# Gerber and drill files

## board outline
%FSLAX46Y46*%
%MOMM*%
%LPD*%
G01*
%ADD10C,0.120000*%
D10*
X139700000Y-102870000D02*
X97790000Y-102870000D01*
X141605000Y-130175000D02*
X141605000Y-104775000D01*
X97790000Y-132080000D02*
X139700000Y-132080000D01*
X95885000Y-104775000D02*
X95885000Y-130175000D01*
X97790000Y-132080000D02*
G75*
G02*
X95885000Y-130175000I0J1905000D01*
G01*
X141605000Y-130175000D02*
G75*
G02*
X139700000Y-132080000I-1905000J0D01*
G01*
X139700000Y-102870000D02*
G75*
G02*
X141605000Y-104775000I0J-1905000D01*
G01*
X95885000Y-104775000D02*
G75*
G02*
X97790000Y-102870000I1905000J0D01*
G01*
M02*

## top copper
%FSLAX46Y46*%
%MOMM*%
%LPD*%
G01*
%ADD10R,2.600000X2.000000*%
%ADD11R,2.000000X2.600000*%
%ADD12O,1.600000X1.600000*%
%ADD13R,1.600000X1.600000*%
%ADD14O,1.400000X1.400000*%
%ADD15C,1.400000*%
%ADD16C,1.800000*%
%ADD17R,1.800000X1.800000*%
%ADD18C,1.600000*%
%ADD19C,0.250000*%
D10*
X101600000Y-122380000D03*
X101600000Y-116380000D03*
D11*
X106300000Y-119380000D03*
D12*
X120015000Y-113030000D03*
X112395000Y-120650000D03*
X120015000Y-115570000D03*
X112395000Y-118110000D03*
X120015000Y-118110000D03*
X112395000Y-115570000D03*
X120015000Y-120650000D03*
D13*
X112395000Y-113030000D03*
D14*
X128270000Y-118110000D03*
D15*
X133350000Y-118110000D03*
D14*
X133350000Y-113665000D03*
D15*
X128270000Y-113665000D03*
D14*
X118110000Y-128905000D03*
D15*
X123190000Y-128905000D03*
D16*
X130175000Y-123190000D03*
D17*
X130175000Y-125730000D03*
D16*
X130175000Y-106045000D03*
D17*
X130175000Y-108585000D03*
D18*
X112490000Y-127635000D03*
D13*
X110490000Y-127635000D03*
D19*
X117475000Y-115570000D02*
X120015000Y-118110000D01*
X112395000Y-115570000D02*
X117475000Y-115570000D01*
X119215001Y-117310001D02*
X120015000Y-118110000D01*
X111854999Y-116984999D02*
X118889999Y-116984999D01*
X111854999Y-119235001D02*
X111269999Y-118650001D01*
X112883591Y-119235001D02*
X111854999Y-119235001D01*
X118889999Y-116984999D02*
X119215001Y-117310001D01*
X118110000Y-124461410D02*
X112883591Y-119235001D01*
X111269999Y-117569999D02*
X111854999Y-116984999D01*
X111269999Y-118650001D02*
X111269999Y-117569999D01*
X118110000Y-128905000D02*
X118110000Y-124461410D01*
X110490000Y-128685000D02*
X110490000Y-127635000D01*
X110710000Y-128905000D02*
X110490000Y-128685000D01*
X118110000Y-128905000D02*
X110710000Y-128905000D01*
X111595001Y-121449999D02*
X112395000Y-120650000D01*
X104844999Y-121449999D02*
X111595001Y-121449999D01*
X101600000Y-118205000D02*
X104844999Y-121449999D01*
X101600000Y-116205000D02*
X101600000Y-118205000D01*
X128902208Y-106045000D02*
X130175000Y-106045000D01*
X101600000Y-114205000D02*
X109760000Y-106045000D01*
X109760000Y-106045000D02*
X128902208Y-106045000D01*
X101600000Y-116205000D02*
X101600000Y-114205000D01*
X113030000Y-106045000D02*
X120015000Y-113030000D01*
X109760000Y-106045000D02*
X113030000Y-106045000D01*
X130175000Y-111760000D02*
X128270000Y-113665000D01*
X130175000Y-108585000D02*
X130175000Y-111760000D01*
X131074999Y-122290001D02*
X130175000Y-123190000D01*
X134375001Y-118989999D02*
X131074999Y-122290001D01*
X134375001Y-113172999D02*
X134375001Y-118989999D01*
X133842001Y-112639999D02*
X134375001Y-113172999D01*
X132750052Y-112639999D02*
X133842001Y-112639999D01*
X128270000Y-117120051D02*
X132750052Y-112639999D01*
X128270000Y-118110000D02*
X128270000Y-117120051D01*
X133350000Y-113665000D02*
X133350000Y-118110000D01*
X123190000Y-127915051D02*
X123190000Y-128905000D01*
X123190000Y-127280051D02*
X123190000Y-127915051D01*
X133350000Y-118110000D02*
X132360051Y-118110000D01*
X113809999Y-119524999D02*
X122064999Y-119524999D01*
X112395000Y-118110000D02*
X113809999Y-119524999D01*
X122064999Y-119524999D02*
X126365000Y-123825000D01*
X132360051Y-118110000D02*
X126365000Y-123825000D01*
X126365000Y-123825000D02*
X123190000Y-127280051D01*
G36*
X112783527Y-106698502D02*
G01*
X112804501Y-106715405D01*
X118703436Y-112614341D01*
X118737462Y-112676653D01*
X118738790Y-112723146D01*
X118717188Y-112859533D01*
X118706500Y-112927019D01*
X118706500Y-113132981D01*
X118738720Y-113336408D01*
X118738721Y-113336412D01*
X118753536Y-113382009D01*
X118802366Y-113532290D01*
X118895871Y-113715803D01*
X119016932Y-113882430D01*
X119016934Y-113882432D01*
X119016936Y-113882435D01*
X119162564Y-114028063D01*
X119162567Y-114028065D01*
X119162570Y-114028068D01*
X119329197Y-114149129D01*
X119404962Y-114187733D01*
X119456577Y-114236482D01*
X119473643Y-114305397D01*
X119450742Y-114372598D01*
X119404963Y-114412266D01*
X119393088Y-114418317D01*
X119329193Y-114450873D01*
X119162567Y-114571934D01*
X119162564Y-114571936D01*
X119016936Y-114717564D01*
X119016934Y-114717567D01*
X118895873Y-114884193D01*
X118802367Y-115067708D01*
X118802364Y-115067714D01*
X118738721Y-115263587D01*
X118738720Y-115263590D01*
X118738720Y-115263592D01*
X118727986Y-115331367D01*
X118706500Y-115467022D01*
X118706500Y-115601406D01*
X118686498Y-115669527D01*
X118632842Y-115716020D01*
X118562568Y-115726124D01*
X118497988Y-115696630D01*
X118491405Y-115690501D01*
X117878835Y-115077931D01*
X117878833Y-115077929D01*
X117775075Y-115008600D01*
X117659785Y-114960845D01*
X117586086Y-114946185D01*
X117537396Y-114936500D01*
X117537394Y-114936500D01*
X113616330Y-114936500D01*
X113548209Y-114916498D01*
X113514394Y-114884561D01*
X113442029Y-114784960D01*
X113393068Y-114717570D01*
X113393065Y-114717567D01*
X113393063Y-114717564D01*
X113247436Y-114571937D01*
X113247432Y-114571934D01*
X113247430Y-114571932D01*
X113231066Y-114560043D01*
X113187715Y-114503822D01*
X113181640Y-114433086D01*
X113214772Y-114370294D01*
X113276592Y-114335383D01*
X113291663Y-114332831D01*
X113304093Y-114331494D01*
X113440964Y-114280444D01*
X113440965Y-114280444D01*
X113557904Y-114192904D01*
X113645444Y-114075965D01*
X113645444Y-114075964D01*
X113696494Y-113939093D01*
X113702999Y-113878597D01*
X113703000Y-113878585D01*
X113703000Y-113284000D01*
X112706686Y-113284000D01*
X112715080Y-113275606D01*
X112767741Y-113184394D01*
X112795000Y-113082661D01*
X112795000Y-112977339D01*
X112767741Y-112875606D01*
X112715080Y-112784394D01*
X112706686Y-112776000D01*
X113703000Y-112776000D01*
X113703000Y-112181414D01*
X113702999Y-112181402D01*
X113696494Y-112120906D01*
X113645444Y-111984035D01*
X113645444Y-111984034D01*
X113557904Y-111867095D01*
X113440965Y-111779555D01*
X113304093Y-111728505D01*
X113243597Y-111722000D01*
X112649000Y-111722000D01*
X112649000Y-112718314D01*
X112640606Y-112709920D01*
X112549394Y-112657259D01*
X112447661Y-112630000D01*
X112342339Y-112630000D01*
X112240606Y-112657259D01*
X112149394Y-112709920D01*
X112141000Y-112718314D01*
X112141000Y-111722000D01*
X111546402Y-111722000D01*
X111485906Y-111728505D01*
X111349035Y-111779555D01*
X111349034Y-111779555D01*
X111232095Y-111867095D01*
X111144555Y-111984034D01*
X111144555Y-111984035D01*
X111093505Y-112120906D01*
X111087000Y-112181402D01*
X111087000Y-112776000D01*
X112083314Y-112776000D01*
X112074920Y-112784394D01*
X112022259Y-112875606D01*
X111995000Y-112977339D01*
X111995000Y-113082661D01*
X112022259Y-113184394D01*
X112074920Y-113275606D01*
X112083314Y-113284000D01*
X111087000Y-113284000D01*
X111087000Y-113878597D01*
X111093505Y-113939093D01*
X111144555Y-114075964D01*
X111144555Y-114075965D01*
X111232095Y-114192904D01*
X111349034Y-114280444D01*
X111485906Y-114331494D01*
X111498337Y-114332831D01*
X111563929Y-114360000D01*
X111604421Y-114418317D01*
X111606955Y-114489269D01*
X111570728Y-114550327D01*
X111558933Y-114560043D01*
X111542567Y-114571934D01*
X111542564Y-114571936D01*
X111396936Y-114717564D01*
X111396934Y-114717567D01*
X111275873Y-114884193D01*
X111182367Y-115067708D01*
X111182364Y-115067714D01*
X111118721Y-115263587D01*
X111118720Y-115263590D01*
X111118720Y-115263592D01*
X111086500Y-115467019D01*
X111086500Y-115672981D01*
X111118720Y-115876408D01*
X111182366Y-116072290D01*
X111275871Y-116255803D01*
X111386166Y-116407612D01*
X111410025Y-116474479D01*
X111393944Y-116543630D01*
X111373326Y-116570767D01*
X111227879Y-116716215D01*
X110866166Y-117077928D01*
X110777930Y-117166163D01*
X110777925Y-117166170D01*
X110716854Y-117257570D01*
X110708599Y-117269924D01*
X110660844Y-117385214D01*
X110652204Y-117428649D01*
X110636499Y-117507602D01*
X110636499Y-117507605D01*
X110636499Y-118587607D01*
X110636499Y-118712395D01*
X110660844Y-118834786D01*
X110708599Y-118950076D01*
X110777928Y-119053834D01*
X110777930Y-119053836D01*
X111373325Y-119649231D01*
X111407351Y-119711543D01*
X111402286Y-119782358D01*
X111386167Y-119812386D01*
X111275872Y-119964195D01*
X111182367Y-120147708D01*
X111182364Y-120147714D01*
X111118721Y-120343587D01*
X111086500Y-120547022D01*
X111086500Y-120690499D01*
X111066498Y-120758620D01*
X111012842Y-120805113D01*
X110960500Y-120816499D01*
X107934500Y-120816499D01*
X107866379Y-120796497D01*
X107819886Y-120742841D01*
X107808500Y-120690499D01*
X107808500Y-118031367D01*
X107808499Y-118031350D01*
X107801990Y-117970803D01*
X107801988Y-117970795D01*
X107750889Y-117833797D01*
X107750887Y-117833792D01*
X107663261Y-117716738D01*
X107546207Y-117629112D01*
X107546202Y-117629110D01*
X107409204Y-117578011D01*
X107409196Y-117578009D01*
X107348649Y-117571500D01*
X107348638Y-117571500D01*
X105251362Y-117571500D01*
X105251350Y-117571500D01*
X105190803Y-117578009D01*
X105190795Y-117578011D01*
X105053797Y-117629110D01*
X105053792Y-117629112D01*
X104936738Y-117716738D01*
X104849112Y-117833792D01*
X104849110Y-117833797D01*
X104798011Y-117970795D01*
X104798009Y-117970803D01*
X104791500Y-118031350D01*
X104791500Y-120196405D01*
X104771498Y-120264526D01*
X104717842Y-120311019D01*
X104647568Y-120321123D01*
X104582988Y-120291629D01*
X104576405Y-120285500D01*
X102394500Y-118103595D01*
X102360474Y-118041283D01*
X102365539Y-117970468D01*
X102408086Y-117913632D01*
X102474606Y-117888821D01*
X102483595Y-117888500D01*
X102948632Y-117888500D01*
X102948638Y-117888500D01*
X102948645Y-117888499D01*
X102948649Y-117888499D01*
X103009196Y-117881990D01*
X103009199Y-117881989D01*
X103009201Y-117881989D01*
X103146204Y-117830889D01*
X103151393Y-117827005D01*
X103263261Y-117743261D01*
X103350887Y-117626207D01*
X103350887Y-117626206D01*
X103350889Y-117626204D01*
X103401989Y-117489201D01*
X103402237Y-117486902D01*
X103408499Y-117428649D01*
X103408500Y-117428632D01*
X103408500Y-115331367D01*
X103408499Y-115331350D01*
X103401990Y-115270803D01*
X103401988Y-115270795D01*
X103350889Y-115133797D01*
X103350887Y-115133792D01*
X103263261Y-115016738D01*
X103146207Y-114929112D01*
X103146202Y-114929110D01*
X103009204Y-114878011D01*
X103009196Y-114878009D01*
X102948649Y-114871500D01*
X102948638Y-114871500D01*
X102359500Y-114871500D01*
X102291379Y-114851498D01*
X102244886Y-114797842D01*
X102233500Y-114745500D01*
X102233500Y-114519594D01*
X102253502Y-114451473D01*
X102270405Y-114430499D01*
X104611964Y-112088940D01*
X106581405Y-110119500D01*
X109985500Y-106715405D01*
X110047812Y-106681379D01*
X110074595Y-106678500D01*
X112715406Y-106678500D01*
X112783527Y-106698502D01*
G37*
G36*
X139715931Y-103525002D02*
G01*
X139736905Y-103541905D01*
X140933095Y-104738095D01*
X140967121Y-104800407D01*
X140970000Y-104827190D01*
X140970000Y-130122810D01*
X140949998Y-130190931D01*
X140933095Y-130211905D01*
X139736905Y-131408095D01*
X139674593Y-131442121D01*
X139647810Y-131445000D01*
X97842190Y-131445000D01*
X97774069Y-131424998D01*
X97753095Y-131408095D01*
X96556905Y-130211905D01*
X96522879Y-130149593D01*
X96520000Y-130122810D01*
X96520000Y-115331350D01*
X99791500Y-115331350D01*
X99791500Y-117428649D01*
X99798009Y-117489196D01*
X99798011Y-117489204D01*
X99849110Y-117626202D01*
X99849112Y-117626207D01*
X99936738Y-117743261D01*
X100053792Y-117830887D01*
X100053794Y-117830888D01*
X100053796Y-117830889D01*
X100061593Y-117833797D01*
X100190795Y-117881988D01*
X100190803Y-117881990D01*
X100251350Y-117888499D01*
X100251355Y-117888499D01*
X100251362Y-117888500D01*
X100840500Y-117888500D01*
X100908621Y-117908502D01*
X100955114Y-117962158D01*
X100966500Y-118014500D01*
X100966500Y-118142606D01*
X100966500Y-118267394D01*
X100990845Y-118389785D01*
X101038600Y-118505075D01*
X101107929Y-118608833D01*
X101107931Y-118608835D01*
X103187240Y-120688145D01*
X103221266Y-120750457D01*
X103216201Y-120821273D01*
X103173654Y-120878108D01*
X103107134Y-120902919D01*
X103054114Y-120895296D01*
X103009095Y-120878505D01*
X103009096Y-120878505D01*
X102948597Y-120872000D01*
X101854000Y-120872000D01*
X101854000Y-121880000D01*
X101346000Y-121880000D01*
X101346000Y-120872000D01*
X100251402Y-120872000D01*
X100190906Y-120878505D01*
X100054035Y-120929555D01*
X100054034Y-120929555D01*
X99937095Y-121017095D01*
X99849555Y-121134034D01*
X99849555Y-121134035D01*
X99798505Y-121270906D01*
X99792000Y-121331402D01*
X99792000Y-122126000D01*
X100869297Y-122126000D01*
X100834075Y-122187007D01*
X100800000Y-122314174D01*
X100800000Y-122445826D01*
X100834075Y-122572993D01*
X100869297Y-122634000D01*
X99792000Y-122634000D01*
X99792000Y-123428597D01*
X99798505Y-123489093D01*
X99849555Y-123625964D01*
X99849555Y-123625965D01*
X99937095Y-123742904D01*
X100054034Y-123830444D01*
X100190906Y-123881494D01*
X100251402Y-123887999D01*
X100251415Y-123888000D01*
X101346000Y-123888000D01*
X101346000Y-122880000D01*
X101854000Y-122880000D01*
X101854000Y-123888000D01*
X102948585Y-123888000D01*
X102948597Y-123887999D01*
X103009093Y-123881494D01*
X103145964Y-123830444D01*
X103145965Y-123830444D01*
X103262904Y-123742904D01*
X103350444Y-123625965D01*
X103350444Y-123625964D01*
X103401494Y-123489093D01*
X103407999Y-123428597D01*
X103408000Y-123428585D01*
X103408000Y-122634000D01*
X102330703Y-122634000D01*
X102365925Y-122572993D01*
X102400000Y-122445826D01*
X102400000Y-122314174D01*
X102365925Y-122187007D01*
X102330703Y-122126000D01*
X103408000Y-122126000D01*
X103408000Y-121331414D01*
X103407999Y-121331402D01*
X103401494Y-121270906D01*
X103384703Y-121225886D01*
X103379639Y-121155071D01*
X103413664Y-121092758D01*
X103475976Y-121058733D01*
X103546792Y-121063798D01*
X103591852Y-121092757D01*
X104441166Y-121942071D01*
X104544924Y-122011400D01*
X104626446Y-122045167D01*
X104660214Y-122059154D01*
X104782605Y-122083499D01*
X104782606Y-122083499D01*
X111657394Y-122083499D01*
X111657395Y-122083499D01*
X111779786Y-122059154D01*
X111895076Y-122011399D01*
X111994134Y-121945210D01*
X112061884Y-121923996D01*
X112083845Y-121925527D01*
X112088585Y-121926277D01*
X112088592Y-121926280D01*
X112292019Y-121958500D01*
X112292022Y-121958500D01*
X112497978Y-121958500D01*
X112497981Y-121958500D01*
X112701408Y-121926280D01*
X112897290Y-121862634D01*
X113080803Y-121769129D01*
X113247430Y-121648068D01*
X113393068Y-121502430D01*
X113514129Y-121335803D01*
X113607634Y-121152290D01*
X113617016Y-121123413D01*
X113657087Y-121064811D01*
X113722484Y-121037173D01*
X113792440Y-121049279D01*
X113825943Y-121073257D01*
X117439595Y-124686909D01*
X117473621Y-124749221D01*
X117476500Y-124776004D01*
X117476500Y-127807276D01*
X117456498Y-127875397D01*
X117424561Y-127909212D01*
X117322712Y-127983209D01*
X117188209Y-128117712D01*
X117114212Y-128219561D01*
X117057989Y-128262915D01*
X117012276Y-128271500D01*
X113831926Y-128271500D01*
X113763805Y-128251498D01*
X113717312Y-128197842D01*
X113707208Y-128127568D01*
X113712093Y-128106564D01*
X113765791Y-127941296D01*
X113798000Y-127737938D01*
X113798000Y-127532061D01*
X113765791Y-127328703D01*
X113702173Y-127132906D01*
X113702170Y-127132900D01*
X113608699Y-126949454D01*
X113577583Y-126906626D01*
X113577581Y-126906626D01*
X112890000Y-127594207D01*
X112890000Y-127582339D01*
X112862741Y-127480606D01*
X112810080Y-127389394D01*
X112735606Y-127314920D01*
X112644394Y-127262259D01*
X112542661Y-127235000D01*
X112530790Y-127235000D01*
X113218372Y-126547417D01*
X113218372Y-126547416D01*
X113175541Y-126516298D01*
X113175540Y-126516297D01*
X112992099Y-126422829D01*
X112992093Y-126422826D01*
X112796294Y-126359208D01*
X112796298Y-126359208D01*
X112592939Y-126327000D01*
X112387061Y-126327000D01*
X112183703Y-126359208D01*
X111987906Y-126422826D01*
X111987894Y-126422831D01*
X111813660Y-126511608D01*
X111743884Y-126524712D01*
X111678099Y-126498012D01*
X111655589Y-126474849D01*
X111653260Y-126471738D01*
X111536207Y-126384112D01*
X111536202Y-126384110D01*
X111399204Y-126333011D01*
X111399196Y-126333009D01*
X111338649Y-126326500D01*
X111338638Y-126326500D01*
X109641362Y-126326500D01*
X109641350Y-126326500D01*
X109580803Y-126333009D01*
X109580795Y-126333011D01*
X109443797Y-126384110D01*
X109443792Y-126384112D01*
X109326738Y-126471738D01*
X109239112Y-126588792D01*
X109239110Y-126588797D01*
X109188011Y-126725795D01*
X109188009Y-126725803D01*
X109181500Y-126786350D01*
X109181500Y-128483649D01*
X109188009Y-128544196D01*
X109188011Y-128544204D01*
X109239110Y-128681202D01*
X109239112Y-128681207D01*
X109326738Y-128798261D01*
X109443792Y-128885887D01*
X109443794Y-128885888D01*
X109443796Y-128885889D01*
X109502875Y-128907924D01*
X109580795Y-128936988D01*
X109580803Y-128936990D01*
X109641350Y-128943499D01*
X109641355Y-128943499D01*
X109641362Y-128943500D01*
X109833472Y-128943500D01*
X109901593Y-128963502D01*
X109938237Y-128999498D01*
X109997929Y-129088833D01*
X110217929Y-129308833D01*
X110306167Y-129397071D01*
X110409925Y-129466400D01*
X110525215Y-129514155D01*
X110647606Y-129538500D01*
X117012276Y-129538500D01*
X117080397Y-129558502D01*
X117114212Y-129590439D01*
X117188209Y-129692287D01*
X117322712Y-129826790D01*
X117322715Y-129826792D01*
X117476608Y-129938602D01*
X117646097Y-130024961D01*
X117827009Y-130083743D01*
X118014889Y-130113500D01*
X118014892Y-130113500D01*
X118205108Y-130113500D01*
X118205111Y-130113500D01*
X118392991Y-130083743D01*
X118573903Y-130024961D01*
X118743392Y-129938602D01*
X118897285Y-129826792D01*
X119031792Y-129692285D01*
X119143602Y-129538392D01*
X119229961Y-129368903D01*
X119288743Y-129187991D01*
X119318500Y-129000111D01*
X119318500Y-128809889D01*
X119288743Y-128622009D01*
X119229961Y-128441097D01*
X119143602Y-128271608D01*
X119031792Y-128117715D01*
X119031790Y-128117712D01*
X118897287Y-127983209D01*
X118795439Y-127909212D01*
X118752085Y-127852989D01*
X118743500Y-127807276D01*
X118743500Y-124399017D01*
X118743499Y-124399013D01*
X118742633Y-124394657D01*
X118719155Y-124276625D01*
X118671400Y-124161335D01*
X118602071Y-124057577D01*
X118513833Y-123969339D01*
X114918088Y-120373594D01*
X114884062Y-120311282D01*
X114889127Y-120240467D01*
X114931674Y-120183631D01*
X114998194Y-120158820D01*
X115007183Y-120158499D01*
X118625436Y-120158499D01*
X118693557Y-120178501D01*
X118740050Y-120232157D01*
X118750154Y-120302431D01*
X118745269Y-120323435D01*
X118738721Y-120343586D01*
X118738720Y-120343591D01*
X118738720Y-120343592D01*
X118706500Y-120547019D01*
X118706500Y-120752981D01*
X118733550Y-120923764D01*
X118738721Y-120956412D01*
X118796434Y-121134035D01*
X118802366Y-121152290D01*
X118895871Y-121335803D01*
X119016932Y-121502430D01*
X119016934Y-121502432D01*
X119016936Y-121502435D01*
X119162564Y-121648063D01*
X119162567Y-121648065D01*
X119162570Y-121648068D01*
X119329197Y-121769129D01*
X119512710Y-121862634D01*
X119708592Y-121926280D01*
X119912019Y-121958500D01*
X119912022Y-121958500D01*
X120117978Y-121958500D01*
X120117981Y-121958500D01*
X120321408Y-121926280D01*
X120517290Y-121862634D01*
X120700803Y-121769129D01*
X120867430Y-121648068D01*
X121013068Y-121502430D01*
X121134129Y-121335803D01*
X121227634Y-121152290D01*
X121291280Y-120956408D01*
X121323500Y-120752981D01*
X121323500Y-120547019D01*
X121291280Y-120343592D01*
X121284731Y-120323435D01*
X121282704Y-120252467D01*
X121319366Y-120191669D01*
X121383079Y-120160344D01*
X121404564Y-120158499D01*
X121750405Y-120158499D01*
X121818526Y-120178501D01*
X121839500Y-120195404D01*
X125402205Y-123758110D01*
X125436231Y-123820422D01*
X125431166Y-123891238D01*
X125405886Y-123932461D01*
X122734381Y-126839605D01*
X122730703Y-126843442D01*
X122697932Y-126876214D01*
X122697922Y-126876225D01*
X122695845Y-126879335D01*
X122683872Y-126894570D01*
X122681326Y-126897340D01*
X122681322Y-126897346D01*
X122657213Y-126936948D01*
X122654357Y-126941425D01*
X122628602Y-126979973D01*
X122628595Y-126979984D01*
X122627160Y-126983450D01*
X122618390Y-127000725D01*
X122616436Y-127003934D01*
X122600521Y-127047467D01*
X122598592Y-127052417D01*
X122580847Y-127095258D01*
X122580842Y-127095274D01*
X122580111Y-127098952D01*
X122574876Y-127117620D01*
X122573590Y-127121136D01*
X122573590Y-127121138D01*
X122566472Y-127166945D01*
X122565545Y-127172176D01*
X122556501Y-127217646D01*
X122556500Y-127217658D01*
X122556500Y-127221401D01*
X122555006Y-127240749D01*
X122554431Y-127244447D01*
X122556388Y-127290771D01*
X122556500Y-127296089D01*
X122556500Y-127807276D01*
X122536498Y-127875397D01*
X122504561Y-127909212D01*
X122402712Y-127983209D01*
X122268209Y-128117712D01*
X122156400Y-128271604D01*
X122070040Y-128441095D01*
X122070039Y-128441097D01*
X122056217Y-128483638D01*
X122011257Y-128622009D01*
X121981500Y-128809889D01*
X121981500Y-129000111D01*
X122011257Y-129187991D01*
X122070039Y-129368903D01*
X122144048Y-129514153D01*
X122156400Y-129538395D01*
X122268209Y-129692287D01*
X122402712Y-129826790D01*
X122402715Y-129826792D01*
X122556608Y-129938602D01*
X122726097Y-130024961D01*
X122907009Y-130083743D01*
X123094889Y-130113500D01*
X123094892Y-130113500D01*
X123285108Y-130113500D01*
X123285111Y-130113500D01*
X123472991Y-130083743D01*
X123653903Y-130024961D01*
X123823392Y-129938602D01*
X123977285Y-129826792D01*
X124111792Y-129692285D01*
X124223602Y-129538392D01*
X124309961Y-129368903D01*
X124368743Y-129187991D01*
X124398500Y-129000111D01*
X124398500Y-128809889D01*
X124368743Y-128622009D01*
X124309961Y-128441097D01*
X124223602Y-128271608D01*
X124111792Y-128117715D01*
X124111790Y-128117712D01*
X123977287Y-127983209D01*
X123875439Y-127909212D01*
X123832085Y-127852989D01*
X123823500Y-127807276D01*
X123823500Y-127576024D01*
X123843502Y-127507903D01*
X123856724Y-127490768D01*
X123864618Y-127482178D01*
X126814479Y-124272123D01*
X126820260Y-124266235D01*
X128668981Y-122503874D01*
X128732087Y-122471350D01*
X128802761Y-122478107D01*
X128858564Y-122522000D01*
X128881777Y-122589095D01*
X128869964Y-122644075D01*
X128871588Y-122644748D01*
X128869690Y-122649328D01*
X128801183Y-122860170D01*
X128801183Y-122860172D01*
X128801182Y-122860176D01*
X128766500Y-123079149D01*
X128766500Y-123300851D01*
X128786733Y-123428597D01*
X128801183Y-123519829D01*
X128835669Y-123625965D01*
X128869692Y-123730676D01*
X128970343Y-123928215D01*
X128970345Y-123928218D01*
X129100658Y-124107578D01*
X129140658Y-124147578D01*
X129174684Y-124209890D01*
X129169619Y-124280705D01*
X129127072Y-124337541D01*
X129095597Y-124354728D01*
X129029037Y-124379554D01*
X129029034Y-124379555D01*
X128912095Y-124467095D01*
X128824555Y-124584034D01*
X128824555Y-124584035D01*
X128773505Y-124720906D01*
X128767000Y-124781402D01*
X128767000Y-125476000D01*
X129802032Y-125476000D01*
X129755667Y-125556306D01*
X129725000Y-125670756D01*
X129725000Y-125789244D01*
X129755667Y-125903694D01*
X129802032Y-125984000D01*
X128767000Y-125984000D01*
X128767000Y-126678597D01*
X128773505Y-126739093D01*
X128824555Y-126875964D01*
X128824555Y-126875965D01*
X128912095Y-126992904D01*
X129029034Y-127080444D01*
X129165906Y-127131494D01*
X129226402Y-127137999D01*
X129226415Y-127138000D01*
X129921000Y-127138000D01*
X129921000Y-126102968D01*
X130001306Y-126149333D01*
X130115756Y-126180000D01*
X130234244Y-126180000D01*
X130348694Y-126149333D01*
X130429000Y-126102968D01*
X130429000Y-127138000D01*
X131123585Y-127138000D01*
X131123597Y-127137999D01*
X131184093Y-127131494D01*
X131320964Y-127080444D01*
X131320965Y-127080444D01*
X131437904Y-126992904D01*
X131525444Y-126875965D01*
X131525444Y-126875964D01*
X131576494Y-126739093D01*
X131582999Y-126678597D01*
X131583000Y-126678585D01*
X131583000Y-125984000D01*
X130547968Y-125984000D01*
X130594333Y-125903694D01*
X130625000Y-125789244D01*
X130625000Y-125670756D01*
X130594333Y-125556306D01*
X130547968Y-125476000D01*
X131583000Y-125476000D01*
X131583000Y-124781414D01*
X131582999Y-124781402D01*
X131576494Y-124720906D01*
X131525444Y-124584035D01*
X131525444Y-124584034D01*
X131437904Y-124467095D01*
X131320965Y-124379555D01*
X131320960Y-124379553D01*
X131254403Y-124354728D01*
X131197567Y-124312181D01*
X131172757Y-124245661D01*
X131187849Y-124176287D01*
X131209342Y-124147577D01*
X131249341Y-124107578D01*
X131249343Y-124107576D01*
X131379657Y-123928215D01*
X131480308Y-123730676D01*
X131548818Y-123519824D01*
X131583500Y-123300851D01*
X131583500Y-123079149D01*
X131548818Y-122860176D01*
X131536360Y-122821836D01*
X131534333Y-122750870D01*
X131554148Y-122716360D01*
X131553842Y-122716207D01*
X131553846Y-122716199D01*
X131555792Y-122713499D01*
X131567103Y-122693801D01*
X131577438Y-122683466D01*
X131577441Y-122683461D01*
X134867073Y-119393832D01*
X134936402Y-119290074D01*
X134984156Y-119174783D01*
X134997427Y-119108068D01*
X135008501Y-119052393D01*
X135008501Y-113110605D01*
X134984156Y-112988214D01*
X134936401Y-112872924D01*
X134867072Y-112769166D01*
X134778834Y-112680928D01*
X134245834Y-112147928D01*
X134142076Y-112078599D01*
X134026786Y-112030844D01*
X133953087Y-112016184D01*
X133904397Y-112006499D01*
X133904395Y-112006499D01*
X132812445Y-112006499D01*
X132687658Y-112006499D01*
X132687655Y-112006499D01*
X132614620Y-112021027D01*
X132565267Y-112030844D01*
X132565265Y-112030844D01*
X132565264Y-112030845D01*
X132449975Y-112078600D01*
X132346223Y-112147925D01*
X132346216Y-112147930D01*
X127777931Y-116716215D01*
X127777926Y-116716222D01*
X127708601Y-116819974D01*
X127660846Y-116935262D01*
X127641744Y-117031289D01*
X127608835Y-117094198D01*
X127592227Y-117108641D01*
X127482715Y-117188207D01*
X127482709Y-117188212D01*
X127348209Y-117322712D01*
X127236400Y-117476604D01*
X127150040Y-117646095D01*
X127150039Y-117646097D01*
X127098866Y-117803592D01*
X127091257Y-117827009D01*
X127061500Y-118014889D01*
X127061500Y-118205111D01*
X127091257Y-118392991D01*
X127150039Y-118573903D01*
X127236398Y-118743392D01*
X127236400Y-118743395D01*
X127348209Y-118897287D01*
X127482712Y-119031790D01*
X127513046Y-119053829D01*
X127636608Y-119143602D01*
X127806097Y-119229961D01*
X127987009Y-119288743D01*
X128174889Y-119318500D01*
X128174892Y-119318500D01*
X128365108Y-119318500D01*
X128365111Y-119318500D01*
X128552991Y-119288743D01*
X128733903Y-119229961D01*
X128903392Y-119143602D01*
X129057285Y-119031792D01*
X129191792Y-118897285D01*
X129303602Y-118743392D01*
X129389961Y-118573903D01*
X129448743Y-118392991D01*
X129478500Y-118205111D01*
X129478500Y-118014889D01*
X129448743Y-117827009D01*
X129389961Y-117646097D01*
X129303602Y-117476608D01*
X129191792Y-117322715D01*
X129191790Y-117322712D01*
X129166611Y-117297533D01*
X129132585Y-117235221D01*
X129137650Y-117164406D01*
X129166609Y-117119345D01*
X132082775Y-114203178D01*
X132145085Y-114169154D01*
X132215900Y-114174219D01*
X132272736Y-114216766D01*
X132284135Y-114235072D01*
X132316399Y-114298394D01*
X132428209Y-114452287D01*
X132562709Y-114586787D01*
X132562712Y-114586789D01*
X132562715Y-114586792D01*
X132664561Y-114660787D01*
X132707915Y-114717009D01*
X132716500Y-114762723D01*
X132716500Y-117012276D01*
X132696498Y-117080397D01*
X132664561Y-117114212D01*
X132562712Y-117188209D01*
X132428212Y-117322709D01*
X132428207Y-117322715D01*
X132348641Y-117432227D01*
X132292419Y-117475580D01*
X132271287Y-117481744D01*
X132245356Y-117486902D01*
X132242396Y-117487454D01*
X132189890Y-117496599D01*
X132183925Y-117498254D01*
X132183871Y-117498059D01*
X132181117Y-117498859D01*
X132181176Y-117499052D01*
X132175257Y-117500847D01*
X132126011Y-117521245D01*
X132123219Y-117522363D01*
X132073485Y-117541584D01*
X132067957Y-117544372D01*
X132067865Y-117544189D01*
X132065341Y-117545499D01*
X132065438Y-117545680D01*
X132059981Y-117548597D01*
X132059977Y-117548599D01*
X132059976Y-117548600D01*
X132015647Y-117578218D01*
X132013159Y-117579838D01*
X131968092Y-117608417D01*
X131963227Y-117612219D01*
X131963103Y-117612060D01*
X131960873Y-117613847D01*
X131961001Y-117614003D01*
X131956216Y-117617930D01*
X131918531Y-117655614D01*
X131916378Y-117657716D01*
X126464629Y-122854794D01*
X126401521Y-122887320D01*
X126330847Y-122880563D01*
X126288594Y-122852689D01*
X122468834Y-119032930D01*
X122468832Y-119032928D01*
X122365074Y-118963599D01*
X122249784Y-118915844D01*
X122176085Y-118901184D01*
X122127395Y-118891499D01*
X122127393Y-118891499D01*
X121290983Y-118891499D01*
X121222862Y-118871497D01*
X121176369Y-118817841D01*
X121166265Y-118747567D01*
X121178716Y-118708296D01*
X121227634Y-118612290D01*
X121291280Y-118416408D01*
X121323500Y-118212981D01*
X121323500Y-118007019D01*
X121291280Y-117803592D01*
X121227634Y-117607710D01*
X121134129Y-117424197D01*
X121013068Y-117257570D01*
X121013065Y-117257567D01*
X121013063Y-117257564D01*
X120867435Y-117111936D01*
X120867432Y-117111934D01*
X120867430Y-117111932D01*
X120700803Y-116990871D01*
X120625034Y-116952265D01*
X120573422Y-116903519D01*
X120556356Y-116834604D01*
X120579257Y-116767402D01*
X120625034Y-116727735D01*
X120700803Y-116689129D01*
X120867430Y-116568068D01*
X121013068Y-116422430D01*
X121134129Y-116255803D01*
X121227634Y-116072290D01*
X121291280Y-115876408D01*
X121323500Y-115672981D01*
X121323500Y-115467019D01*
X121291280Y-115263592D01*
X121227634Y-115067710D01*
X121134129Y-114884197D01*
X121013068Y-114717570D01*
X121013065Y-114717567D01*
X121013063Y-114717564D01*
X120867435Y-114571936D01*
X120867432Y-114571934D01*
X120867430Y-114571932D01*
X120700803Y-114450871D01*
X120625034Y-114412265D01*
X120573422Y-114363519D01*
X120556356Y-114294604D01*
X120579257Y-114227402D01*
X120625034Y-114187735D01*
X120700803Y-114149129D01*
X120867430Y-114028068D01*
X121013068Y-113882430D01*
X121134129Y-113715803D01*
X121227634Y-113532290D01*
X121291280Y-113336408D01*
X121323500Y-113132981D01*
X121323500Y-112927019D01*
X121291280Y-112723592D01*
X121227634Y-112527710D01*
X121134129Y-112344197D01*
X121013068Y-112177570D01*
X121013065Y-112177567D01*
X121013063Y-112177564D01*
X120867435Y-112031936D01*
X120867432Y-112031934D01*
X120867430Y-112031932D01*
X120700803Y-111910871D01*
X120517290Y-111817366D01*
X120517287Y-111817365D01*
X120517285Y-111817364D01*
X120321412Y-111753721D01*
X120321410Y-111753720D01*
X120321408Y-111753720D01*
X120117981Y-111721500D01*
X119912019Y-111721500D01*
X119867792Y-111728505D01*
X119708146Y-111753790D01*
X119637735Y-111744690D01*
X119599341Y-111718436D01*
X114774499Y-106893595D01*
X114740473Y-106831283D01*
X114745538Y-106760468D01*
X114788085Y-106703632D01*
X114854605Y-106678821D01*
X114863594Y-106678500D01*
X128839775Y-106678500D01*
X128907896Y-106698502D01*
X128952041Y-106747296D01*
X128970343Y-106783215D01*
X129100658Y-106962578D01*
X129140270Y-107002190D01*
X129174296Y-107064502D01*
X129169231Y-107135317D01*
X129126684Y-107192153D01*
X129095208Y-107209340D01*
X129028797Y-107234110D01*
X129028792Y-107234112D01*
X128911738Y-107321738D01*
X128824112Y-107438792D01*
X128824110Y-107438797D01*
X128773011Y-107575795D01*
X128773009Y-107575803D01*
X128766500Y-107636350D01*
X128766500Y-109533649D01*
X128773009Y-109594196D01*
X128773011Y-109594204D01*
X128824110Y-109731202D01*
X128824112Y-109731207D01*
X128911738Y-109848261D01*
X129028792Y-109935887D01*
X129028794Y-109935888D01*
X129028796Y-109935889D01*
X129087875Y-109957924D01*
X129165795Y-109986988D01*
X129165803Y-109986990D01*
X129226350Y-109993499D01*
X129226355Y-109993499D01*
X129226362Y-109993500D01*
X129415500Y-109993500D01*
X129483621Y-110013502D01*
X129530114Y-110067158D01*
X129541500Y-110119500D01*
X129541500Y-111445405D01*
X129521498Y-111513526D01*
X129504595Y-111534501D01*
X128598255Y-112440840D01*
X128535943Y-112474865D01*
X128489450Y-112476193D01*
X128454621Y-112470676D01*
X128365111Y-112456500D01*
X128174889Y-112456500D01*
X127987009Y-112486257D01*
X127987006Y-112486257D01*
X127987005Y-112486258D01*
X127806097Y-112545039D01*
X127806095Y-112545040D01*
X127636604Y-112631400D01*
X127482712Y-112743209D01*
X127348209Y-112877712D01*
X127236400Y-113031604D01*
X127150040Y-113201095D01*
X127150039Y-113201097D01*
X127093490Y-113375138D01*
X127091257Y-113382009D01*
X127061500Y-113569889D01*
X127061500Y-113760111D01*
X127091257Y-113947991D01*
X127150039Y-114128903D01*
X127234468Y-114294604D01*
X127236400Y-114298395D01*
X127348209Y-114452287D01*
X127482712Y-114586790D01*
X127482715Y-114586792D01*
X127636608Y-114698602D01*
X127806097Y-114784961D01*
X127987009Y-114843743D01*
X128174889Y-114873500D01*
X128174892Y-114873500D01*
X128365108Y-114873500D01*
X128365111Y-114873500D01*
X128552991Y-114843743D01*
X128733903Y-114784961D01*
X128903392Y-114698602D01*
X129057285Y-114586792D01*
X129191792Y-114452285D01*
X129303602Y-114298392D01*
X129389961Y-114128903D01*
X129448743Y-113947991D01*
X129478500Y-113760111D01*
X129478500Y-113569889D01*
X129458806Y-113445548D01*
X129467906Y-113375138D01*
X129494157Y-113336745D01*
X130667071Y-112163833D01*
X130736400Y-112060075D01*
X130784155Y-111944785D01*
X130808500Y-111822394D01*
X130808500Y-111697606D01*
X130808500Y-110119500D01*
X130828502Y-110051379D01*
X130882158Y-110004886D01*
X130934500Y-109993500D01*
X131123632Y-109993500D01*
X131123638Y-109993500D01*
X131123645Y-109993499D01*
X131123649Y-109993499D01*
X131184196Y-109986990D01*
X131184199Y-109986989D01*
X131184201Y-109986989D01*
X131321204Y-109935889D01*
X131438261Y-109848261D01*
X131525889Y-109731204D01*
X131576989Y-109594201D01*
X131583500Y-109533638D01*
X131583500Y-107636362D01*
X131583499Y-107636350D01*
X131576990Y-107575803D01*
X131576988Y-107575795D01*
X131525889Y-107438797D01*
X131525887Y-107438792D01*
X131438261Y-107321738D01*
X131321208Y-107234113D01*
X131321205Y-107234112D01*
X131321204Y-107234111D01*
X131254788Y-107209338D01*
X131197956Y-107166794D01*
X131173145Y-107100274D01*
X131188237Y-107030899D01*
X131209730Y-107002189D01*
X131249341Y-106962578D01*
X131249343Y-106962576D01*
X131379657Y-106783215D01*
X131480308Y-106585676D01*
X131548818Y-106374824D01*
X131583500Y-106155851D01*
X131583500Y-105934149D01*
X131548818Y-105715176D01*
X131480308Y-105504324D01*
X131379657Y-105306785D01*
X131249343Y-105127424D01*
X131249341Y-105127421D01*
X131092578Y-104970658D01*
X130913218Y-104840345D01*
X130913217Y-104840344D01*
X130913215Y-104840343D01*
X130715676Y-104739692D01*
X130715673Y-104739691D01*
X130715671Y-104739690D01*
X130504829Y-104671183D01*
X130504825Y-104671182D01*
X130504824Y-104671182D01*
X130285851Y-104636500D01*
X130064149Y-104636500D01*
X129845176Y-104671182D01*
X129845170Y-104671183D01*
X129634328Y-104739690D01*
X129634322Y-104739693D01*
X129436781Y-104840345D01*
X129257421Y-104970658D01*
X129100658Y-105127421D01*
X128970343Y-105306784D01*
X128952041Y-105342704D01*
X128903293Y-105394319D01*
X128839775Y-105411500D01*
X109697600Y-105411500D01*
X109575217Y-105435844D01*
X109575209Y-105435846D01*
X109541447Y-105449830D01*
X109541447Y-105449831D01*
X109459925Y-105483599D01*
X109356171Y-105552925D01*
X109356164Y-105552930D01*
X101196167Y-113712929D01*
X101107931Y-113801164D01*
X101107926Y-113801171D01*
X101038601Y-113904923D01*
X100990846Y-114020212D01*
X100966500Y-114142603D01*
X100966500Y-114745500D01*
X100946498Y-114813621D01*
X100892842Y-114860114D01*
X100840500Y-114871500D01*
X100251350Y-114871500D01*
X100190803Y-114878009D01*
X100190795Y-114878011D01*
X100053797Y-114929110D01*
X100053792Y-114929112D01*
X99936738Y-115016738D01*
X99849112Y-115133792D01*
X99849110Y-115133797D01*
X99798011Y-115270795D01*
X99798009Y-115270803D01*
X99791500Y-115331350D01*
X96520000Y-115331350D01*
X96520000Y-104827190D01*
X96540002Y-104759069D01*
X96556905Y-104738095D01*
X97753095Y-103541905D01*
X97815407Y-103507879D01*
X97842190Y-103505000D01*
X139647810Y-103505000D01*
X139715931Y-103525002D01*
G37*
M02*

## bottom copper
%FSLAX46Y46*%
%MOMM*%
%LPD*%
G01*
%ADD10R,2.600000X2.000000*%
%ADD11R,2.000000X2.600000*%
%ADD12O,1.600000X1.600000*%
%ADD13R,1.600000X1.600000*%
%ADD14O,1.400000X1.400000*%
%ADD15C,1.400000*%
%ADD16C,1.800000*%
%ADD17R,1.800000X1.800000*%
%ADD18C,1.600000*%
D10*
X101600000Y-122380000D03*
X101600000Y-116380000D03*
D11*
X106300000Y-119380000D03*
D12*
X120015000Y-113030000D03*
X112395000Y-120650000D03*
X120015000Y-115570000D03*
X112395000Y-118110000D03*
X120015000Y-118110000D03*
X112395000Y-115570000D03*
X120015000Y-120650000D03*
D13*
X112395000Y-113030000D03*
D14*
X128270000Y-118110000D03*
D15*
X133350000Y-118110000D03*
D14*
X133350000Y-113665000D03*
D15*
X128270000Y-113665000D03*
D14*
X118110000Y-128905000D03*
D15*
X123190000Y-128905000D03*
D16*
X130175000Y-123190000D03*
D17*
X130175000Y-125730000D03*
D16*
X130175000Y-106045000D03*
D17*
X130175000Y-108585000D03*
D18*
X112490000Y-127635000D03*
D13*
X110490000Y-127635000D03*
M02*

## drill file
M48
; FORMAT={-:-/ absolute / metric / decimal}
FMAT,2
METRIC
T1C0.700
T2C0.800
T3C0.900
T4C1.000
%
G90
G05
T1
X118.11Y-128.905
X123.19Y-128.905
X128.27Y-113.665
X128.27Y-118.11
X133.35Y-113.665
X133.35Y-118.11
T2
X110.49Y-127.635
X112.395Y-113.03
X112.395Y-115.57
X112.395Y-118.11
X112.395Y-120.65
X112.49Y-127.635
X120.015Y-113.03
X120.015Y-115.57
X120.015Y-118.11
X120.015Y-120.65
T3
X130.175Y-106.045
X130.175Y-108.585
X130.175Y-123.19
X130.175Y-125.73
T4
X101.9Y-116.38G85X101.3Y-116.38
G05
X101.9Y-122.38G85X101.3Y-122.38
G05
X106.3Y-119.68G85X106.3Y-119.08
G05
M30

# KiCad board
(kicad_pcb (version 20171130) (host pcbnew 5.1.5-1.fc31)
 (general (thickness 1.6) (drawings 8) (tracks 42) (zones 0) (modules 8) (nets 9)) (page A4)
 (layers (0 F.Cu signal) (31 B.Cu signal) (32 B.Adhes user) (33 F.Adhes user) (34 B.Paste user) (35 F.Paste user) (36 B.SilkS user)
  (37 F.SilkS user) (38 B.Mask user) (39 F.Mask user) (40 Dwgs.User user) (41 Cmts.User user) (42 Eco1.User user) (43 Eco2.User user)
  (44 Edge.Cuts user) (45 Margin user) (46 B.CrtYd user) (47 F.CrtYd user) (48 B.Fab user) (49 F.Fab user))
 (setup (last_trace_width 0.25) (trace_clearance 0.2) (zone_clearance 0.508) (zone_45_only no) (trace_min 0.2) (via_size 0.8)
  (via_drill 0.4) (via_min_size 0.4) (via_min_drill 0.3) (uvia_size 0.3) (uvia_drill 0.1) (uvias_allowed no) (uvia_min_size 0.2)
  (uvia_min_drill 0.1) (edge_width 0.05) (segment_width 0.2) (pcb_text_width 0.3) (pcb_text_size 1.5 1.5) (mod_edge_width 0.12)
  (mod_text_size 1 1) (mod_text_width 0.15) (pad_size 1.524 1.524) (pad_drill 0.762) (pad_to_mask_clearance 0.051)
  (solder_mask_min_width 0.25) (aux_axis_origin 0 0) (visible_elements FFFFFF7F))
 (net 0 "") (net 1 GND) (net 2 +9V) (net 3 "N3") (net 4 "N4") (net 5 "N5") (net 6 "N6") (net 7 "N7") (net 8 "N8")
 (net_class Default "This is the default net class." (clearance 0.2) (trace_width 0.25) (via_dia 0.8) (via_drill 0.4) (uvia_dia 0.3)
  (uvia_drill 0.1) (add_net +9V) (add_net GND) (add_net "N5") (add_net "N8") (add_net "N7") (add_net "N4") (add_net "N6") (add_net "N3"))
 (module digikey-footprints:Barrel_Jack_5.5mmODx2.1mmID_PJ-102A (layer F.Cu) (at 101.6 119.38 180)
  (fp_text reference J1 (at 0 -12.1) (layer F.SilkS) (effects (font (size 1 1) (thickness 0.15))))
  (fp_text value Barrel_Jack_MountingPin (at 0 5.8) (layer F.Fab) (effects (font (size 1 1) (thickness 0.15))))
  (pad 2 thru_hole rect (at 0 -3 180) (size 2.6 2) (drill oval 1.6 1) (layers *.Cu *.Mask) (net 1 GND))
  (pad 1 thru_hole rect (at 0 3 180) (size 2.6 2) (drill oval 1.6 1) (layers *.Cu *.Mask) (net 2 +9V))
  (pad 3 thru_hole rect (at -4.7 0 180) (size 2 2.6) (drill oval 1 1.6) (layers *.Cu *.Mask)))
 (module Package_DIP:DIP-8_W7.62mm (layer F.Cu) (at 112.395 113.03)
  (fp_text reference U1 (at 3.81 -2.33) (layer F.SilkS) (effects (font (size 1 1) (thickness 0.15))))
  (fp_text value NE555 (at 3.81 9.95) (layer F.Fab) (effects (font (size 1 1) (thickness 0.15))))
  (pad 8 thru_hole oval (at 7.62 0) (size 1.6 1.6) (drill 0.8) (layers *.Cu *.Mask) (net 2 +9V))
  (pad 4 thru_hole oval (at 0 7.62) (size 1.6 1.6) (drill 0.8) (layers *.Cu *.Mask) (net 2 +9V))
  (pad 7 thru_hole oval (at 7.62 2.54) (size 1.6 1.6) (drill 0.8) (layers *.Cu *.Mask) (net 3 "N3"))
  (pad 3 thru_hole oval (at 0 5.08) (size 1.6 1.6) (drill 0.8) (layers *.Cu *.Mask) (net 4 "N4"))
  (pad 6 thru_hole oval (at 7.62 5.08) (size 1.6 1.6) (drill 0.8) (layers *.Cu *.Mask) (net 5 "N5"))
  (pad 2 thru_hole oval (at 0 2.54) (size 1.6 1.6) (drill 0.8) (layers *.Cu *.Mask) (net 5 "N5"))
  (pad 5 thru_hole oval (at 7.62 7.62) (size 1.6 1.6) (drill 0.8) (layers *.Cu *.Mask) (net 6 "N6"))
  (pad 1 thru_hole rect (at 0 0) (size 1.6 1.6) (drill 0.8) (layers *.Cu *.Mask) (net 1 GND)))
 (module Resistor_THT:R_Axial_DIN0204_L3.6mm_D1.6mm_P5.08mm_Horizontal (layer F.Cu) (at 133.35 118.11 180)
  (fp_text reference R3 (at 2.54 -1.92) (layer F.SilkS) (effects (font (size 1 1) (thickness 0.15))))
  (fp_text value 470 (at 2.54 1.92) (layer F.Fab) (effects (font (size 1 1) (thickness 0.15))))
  (pad 2 thru_hole oval (at 5.08 0 180) (size 1.4 1.4) (drill 0.7) (layers *.Cu *.Mask) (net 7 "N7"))
  (pad 1 thru_hole circle (at 0 0 180) (size 1.4 1.4) (drill 0.7) (layers *.Cu *.Mask) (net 4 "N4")))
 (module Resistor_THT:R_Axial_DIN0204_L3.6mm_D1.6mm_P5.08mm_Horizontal (layer F.Cu) (at 128.27 113.665)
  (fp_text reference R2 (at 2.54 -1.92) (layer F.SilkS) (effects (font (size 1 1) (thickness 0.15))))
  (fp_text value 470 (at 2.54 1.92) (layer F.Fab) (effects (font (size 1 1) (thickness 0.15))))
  (pad 2 thru_hole oval (at 5.08 0) (size 1.4 1.4) (drill 0.7) (layers *.Cu *.Mask) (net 4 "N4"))
  (pad 1 thru_hole circle (at 0 0) (size 1.4 1.4) (drill 0.7) (layers *.Cu *.Mask) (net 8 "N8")))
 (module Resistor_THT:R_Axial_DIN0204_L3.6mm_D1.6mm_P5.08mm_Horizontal (layer F.Cu) (at 123.19 128.905 180)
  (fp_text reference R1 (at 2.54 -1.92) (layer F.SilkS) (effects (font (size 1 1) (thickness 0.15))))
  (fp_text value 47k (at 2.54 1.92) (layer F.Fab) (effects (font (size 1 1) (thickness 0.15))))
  (pad 2 thru_hole oval (at 5.08 0 180) (size 1.4 1.4) (drill 0.7) (layers *.Cu *.Mask) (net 5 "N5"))
  (pad 1 thru_hole circle (at 0 0 180) (size 1.4 1.4) (drill 0.7) (layers *.Cu *.Mask) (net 4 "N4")))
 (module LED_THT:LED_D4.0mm (layer F.Cu) (at 130.175 125.73 90)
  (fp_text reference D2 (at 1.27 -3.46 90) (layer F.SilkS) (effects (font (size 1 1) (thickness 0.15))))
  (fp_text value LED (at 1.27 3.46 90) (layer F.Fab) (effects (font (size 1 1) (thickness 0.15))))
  (pad 2 thru_hole circle (at 2.54 0 90) (size 1.8 1.8) (drill 0.9) (layers *.Cu *.Mask) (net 7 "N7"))
  (pad 1 thru_hole rect (at 0 0 90) (size 1.8 1.8) (drill 0.9) (layers *.Cu *.Mask) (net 1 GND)))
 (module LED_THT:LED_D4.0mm (layer F.Cu) (at 130.175 108.585 90)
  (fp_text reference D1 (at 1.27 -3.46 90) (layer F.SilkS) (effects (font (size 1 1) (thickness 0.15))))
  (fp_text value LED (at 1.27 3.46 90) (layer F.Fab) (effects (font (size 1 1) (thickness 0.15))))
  (pad 2 thru_hole circle (at 2.54 0 90) (size 1.8 1.8) (drill 0.9) (layers *.Cu *.Mask) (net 2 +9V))
  (pad 1 thru_hole rect (at 0 0 90) (size 1.8 1.8) (drill 0.9) (layers *.Cu *.Mask) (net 8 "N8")))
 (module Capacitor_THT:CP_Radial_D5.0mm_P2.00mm (layer F.Cu) (at 110.49 127.635)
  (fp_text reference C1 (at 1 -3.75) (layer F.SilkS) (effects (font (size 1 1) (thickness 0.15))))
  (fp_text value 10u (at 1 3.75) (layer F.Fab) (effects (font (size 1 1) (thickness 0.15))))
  (pad 2 thru_hole circle (at 2 0) (size 1.6 1.6) (drill 0.8) (layers *.Cu *.Mask) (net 1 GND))
  (pad 1 thru_hole rect (at 0 0) (size 1.6 1.6) (drill 0.8) (layers *.Cu *.Mask) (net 5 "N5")))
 (gr_line (start 139.7 102.87) (end 97.79 102.87) (layer Edge.Cuts) (width 0.12))
 (gr_line (start 141.605 130.175) (end 141.605 104.775) (layer Edge.Cuts) (width 0.12))
 (gr_line (start 97.79 132.08) (end 139.7 132.08) (layer Edge.Cuts) (width 0.12))
 (gr_line (start 95.885 104.775) (end 95.885 130.175) (layer Edge.Cuts) (width 0.12))
 (gr_arc (start 97.79 130.175) (end 95.885 130.175) (angle -90) (layer Edge.Cuts) (width 0.12))
 (gr_arc (start 139.7 130.175) (end 139.7 132.08) (angle -90) (layer Edge.Cuts) (width 0.12))
 (gr_arc (start 139.7 104.775) (end 141.605 104.775) (angle -90) (layer Edge.Cuts) (width 0.12))
 (gr_arc (start 97.79 104.775) (end 97.79 102.87) (angle -90) (layer Edge.Cuts) (width 0.12))
 (segment (start 117.475 115.57) (end 120.015 118.11) (width 0.25) (layer F.Cu) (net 5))
 (segment (start 112.395 115.57) (end 117.475 115.57) (width 0.25) (layer F.Cu) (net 5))
 (segment (start 119.215001 117.310001) (end 120.015 118.11) (width 0.25) (layer F.Cu) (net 5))
 (segment (start 111.854999 116.984999) (end 118.889999 116.984999) (width 0.25) (layer F.Cu) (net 5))
 (segment (start 111.854999 119.235001) (end 111.269999 118.650001) (width 0.25) (layer F.Cu) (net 5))
 (segment (start 112.883591 119.235001) (end 111.854999 119.235001) (width 0.25) (layer F.Cu) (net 5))
 (segment (start 118.889999 116.984999) (end 119.215001 117.310001) (width 0.25) (layer F.Cu) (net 5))
 (segment (start 118.11 124.46141) (end 112.883591 119.235001) (width 0.25) (layer F.Cu) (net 5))
 (segment (start 111.269999 117.569999) (end 111.854999 116.984999) (width 0.25) (layer F.Cu) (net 5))
 (segment (start 111.269999 118.650001) (end 111.269999 117.569999) (width 0.25) (layer F.Cu) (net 5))
 (segment (start 118.11 128.905) (end 118.11 124.46141) (width 0.25) (layer F.Cu) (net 5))
 (segment (start 110.49 128.685) (end 110.49 127.635) (width 0.25) (layer F.Cu) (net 5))
 (segment (start 110.71 128.905) (end 110.49 128.685) (width 0.25) (layer F.Cu) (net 5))
 (segment (start 118.11 128.905) (end 110.71 128.905) (width 0.25) (layer F.Cu) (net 5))
 (segment (start 111.595001 121.449999) (end 112.395 120.65) (width 0.25) (layer F.Cu) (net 2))
 (segment (start 104.844999 121.449999) (end 111.595001 121.449999) (width 0.25) (layer F.Cu) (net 2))
 (segment (start 101.6 118.205) (end 104.844999 121.449999) (width 0.25) (layer F.Cu) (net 2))
 (segment (start 101.6 116.205) (end 101.6 118.205) (width 0.25) (layer F.Cu) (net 2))
 (segment (start 128.902208 106.045) (end 130.175 106.045) (width 0.25) (layer F.Cu) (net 2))
 (segment (start 101.6 114.205) (end 109.76 106.045) (width 0.25) (layer F.Cu) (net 2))
 (segment (start 109.76 106.045) (end 128.902208 106.045) (width 0.25) (layer F.Cu) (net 2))
 (segment (start 101.6 116.205) (end 101.6 114.205) (width 0.25) (layer F.Cu) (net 2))
 (segment (start 113.03 106.045) (end 120.015 113.03) (width 0.25) (layer F.Cu) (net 2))
 (segment (start 109.76 106.045) (end 113.03 106.045) (width 0.25) (layer F.Cu) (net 2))
 (segment (start 130.175 111.76) (end 128.27 113.665) (width 0.25) (layer F.Cu) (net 8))
 (segment (start 130.175 108.585) (end 130.175 111.76) (width 0.25) (layer F.Cu) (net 8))
 (segment (start 131.074999 122.290001) (end 130.175 123.19) (width 0.25) (layer F.Cu) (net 7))
 (segment (start 134.375001 118.989999) (end 131.074999 122.290001) (width 0.25) (layer F.Cu) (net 7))
 (segment (start 134.375001 113.172999) (end 134.375001 118.989999) (width 0.25) (layer F.Cu) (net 7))
 (segment (start 133.842001 112.639999) (end 134.375001 113.172999) (width 0.25) (layer F.Cu) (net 7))
 (segment (start 132.750052 112.639999) (end 133.842001 112.639999) (width 0.25) (layer F.Cu) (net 7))
 (segment (start 128.27 117.120051) (end 132.750052 112.639999) (width 0.25) (layer F.Cu) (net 7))
 (segment (start 128.27 118.11) (end 128.27 117.120051) (width 0.25) (layer F.Cu) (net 7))
 (segment (start 133.35 113.665) (end 133.35 118.11) (width 0.25) (layer F.Cu) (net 4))
 (segment (start 123.19 127.915051) (end 123.19 128.905) (width 0.25) (layer F.Cu) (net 4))
 (segment (start 123.19 127.280051) (end 123.19 127.915051) (width 0.25) (layer F.Cu) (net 4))
 (segment (start 133.35 118.11) (end 132.360051 118.11) (width 0.25) (layer F.Cu) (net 4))
 (segment (start 113.809999 119.524999) (end 122.064999 119.524999) (width 0.25) (layer F.Cu) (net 4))
 (segment (start 112.395 118.11) (end 113.809999 119.524999) (width 0.25) (layer F.Cu) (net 4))
 (segment (start 122.064999 119.524999) (end 126.365 123.825) (width 0.25) (layer F.Cu) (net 4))
 (segment (start 132.360051 118.11) (end 126.365 123.825) (width 0.25) (layer F.Cu) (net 4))
 (segment (start 126.365 123.825) (end 123.19 127.280051) (width 0.25) (layer F.Cu) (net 4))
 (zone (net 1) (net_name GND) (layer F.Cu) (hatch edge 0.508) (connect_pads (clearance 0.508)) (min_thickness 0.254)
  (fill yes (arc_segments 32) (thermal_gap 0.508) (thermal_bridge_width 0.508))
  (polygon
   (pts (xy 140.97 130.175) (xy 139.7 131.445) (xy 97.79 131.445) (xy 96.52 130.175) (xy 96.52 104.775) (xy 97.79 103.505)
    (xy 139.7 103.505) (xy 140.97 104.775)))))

